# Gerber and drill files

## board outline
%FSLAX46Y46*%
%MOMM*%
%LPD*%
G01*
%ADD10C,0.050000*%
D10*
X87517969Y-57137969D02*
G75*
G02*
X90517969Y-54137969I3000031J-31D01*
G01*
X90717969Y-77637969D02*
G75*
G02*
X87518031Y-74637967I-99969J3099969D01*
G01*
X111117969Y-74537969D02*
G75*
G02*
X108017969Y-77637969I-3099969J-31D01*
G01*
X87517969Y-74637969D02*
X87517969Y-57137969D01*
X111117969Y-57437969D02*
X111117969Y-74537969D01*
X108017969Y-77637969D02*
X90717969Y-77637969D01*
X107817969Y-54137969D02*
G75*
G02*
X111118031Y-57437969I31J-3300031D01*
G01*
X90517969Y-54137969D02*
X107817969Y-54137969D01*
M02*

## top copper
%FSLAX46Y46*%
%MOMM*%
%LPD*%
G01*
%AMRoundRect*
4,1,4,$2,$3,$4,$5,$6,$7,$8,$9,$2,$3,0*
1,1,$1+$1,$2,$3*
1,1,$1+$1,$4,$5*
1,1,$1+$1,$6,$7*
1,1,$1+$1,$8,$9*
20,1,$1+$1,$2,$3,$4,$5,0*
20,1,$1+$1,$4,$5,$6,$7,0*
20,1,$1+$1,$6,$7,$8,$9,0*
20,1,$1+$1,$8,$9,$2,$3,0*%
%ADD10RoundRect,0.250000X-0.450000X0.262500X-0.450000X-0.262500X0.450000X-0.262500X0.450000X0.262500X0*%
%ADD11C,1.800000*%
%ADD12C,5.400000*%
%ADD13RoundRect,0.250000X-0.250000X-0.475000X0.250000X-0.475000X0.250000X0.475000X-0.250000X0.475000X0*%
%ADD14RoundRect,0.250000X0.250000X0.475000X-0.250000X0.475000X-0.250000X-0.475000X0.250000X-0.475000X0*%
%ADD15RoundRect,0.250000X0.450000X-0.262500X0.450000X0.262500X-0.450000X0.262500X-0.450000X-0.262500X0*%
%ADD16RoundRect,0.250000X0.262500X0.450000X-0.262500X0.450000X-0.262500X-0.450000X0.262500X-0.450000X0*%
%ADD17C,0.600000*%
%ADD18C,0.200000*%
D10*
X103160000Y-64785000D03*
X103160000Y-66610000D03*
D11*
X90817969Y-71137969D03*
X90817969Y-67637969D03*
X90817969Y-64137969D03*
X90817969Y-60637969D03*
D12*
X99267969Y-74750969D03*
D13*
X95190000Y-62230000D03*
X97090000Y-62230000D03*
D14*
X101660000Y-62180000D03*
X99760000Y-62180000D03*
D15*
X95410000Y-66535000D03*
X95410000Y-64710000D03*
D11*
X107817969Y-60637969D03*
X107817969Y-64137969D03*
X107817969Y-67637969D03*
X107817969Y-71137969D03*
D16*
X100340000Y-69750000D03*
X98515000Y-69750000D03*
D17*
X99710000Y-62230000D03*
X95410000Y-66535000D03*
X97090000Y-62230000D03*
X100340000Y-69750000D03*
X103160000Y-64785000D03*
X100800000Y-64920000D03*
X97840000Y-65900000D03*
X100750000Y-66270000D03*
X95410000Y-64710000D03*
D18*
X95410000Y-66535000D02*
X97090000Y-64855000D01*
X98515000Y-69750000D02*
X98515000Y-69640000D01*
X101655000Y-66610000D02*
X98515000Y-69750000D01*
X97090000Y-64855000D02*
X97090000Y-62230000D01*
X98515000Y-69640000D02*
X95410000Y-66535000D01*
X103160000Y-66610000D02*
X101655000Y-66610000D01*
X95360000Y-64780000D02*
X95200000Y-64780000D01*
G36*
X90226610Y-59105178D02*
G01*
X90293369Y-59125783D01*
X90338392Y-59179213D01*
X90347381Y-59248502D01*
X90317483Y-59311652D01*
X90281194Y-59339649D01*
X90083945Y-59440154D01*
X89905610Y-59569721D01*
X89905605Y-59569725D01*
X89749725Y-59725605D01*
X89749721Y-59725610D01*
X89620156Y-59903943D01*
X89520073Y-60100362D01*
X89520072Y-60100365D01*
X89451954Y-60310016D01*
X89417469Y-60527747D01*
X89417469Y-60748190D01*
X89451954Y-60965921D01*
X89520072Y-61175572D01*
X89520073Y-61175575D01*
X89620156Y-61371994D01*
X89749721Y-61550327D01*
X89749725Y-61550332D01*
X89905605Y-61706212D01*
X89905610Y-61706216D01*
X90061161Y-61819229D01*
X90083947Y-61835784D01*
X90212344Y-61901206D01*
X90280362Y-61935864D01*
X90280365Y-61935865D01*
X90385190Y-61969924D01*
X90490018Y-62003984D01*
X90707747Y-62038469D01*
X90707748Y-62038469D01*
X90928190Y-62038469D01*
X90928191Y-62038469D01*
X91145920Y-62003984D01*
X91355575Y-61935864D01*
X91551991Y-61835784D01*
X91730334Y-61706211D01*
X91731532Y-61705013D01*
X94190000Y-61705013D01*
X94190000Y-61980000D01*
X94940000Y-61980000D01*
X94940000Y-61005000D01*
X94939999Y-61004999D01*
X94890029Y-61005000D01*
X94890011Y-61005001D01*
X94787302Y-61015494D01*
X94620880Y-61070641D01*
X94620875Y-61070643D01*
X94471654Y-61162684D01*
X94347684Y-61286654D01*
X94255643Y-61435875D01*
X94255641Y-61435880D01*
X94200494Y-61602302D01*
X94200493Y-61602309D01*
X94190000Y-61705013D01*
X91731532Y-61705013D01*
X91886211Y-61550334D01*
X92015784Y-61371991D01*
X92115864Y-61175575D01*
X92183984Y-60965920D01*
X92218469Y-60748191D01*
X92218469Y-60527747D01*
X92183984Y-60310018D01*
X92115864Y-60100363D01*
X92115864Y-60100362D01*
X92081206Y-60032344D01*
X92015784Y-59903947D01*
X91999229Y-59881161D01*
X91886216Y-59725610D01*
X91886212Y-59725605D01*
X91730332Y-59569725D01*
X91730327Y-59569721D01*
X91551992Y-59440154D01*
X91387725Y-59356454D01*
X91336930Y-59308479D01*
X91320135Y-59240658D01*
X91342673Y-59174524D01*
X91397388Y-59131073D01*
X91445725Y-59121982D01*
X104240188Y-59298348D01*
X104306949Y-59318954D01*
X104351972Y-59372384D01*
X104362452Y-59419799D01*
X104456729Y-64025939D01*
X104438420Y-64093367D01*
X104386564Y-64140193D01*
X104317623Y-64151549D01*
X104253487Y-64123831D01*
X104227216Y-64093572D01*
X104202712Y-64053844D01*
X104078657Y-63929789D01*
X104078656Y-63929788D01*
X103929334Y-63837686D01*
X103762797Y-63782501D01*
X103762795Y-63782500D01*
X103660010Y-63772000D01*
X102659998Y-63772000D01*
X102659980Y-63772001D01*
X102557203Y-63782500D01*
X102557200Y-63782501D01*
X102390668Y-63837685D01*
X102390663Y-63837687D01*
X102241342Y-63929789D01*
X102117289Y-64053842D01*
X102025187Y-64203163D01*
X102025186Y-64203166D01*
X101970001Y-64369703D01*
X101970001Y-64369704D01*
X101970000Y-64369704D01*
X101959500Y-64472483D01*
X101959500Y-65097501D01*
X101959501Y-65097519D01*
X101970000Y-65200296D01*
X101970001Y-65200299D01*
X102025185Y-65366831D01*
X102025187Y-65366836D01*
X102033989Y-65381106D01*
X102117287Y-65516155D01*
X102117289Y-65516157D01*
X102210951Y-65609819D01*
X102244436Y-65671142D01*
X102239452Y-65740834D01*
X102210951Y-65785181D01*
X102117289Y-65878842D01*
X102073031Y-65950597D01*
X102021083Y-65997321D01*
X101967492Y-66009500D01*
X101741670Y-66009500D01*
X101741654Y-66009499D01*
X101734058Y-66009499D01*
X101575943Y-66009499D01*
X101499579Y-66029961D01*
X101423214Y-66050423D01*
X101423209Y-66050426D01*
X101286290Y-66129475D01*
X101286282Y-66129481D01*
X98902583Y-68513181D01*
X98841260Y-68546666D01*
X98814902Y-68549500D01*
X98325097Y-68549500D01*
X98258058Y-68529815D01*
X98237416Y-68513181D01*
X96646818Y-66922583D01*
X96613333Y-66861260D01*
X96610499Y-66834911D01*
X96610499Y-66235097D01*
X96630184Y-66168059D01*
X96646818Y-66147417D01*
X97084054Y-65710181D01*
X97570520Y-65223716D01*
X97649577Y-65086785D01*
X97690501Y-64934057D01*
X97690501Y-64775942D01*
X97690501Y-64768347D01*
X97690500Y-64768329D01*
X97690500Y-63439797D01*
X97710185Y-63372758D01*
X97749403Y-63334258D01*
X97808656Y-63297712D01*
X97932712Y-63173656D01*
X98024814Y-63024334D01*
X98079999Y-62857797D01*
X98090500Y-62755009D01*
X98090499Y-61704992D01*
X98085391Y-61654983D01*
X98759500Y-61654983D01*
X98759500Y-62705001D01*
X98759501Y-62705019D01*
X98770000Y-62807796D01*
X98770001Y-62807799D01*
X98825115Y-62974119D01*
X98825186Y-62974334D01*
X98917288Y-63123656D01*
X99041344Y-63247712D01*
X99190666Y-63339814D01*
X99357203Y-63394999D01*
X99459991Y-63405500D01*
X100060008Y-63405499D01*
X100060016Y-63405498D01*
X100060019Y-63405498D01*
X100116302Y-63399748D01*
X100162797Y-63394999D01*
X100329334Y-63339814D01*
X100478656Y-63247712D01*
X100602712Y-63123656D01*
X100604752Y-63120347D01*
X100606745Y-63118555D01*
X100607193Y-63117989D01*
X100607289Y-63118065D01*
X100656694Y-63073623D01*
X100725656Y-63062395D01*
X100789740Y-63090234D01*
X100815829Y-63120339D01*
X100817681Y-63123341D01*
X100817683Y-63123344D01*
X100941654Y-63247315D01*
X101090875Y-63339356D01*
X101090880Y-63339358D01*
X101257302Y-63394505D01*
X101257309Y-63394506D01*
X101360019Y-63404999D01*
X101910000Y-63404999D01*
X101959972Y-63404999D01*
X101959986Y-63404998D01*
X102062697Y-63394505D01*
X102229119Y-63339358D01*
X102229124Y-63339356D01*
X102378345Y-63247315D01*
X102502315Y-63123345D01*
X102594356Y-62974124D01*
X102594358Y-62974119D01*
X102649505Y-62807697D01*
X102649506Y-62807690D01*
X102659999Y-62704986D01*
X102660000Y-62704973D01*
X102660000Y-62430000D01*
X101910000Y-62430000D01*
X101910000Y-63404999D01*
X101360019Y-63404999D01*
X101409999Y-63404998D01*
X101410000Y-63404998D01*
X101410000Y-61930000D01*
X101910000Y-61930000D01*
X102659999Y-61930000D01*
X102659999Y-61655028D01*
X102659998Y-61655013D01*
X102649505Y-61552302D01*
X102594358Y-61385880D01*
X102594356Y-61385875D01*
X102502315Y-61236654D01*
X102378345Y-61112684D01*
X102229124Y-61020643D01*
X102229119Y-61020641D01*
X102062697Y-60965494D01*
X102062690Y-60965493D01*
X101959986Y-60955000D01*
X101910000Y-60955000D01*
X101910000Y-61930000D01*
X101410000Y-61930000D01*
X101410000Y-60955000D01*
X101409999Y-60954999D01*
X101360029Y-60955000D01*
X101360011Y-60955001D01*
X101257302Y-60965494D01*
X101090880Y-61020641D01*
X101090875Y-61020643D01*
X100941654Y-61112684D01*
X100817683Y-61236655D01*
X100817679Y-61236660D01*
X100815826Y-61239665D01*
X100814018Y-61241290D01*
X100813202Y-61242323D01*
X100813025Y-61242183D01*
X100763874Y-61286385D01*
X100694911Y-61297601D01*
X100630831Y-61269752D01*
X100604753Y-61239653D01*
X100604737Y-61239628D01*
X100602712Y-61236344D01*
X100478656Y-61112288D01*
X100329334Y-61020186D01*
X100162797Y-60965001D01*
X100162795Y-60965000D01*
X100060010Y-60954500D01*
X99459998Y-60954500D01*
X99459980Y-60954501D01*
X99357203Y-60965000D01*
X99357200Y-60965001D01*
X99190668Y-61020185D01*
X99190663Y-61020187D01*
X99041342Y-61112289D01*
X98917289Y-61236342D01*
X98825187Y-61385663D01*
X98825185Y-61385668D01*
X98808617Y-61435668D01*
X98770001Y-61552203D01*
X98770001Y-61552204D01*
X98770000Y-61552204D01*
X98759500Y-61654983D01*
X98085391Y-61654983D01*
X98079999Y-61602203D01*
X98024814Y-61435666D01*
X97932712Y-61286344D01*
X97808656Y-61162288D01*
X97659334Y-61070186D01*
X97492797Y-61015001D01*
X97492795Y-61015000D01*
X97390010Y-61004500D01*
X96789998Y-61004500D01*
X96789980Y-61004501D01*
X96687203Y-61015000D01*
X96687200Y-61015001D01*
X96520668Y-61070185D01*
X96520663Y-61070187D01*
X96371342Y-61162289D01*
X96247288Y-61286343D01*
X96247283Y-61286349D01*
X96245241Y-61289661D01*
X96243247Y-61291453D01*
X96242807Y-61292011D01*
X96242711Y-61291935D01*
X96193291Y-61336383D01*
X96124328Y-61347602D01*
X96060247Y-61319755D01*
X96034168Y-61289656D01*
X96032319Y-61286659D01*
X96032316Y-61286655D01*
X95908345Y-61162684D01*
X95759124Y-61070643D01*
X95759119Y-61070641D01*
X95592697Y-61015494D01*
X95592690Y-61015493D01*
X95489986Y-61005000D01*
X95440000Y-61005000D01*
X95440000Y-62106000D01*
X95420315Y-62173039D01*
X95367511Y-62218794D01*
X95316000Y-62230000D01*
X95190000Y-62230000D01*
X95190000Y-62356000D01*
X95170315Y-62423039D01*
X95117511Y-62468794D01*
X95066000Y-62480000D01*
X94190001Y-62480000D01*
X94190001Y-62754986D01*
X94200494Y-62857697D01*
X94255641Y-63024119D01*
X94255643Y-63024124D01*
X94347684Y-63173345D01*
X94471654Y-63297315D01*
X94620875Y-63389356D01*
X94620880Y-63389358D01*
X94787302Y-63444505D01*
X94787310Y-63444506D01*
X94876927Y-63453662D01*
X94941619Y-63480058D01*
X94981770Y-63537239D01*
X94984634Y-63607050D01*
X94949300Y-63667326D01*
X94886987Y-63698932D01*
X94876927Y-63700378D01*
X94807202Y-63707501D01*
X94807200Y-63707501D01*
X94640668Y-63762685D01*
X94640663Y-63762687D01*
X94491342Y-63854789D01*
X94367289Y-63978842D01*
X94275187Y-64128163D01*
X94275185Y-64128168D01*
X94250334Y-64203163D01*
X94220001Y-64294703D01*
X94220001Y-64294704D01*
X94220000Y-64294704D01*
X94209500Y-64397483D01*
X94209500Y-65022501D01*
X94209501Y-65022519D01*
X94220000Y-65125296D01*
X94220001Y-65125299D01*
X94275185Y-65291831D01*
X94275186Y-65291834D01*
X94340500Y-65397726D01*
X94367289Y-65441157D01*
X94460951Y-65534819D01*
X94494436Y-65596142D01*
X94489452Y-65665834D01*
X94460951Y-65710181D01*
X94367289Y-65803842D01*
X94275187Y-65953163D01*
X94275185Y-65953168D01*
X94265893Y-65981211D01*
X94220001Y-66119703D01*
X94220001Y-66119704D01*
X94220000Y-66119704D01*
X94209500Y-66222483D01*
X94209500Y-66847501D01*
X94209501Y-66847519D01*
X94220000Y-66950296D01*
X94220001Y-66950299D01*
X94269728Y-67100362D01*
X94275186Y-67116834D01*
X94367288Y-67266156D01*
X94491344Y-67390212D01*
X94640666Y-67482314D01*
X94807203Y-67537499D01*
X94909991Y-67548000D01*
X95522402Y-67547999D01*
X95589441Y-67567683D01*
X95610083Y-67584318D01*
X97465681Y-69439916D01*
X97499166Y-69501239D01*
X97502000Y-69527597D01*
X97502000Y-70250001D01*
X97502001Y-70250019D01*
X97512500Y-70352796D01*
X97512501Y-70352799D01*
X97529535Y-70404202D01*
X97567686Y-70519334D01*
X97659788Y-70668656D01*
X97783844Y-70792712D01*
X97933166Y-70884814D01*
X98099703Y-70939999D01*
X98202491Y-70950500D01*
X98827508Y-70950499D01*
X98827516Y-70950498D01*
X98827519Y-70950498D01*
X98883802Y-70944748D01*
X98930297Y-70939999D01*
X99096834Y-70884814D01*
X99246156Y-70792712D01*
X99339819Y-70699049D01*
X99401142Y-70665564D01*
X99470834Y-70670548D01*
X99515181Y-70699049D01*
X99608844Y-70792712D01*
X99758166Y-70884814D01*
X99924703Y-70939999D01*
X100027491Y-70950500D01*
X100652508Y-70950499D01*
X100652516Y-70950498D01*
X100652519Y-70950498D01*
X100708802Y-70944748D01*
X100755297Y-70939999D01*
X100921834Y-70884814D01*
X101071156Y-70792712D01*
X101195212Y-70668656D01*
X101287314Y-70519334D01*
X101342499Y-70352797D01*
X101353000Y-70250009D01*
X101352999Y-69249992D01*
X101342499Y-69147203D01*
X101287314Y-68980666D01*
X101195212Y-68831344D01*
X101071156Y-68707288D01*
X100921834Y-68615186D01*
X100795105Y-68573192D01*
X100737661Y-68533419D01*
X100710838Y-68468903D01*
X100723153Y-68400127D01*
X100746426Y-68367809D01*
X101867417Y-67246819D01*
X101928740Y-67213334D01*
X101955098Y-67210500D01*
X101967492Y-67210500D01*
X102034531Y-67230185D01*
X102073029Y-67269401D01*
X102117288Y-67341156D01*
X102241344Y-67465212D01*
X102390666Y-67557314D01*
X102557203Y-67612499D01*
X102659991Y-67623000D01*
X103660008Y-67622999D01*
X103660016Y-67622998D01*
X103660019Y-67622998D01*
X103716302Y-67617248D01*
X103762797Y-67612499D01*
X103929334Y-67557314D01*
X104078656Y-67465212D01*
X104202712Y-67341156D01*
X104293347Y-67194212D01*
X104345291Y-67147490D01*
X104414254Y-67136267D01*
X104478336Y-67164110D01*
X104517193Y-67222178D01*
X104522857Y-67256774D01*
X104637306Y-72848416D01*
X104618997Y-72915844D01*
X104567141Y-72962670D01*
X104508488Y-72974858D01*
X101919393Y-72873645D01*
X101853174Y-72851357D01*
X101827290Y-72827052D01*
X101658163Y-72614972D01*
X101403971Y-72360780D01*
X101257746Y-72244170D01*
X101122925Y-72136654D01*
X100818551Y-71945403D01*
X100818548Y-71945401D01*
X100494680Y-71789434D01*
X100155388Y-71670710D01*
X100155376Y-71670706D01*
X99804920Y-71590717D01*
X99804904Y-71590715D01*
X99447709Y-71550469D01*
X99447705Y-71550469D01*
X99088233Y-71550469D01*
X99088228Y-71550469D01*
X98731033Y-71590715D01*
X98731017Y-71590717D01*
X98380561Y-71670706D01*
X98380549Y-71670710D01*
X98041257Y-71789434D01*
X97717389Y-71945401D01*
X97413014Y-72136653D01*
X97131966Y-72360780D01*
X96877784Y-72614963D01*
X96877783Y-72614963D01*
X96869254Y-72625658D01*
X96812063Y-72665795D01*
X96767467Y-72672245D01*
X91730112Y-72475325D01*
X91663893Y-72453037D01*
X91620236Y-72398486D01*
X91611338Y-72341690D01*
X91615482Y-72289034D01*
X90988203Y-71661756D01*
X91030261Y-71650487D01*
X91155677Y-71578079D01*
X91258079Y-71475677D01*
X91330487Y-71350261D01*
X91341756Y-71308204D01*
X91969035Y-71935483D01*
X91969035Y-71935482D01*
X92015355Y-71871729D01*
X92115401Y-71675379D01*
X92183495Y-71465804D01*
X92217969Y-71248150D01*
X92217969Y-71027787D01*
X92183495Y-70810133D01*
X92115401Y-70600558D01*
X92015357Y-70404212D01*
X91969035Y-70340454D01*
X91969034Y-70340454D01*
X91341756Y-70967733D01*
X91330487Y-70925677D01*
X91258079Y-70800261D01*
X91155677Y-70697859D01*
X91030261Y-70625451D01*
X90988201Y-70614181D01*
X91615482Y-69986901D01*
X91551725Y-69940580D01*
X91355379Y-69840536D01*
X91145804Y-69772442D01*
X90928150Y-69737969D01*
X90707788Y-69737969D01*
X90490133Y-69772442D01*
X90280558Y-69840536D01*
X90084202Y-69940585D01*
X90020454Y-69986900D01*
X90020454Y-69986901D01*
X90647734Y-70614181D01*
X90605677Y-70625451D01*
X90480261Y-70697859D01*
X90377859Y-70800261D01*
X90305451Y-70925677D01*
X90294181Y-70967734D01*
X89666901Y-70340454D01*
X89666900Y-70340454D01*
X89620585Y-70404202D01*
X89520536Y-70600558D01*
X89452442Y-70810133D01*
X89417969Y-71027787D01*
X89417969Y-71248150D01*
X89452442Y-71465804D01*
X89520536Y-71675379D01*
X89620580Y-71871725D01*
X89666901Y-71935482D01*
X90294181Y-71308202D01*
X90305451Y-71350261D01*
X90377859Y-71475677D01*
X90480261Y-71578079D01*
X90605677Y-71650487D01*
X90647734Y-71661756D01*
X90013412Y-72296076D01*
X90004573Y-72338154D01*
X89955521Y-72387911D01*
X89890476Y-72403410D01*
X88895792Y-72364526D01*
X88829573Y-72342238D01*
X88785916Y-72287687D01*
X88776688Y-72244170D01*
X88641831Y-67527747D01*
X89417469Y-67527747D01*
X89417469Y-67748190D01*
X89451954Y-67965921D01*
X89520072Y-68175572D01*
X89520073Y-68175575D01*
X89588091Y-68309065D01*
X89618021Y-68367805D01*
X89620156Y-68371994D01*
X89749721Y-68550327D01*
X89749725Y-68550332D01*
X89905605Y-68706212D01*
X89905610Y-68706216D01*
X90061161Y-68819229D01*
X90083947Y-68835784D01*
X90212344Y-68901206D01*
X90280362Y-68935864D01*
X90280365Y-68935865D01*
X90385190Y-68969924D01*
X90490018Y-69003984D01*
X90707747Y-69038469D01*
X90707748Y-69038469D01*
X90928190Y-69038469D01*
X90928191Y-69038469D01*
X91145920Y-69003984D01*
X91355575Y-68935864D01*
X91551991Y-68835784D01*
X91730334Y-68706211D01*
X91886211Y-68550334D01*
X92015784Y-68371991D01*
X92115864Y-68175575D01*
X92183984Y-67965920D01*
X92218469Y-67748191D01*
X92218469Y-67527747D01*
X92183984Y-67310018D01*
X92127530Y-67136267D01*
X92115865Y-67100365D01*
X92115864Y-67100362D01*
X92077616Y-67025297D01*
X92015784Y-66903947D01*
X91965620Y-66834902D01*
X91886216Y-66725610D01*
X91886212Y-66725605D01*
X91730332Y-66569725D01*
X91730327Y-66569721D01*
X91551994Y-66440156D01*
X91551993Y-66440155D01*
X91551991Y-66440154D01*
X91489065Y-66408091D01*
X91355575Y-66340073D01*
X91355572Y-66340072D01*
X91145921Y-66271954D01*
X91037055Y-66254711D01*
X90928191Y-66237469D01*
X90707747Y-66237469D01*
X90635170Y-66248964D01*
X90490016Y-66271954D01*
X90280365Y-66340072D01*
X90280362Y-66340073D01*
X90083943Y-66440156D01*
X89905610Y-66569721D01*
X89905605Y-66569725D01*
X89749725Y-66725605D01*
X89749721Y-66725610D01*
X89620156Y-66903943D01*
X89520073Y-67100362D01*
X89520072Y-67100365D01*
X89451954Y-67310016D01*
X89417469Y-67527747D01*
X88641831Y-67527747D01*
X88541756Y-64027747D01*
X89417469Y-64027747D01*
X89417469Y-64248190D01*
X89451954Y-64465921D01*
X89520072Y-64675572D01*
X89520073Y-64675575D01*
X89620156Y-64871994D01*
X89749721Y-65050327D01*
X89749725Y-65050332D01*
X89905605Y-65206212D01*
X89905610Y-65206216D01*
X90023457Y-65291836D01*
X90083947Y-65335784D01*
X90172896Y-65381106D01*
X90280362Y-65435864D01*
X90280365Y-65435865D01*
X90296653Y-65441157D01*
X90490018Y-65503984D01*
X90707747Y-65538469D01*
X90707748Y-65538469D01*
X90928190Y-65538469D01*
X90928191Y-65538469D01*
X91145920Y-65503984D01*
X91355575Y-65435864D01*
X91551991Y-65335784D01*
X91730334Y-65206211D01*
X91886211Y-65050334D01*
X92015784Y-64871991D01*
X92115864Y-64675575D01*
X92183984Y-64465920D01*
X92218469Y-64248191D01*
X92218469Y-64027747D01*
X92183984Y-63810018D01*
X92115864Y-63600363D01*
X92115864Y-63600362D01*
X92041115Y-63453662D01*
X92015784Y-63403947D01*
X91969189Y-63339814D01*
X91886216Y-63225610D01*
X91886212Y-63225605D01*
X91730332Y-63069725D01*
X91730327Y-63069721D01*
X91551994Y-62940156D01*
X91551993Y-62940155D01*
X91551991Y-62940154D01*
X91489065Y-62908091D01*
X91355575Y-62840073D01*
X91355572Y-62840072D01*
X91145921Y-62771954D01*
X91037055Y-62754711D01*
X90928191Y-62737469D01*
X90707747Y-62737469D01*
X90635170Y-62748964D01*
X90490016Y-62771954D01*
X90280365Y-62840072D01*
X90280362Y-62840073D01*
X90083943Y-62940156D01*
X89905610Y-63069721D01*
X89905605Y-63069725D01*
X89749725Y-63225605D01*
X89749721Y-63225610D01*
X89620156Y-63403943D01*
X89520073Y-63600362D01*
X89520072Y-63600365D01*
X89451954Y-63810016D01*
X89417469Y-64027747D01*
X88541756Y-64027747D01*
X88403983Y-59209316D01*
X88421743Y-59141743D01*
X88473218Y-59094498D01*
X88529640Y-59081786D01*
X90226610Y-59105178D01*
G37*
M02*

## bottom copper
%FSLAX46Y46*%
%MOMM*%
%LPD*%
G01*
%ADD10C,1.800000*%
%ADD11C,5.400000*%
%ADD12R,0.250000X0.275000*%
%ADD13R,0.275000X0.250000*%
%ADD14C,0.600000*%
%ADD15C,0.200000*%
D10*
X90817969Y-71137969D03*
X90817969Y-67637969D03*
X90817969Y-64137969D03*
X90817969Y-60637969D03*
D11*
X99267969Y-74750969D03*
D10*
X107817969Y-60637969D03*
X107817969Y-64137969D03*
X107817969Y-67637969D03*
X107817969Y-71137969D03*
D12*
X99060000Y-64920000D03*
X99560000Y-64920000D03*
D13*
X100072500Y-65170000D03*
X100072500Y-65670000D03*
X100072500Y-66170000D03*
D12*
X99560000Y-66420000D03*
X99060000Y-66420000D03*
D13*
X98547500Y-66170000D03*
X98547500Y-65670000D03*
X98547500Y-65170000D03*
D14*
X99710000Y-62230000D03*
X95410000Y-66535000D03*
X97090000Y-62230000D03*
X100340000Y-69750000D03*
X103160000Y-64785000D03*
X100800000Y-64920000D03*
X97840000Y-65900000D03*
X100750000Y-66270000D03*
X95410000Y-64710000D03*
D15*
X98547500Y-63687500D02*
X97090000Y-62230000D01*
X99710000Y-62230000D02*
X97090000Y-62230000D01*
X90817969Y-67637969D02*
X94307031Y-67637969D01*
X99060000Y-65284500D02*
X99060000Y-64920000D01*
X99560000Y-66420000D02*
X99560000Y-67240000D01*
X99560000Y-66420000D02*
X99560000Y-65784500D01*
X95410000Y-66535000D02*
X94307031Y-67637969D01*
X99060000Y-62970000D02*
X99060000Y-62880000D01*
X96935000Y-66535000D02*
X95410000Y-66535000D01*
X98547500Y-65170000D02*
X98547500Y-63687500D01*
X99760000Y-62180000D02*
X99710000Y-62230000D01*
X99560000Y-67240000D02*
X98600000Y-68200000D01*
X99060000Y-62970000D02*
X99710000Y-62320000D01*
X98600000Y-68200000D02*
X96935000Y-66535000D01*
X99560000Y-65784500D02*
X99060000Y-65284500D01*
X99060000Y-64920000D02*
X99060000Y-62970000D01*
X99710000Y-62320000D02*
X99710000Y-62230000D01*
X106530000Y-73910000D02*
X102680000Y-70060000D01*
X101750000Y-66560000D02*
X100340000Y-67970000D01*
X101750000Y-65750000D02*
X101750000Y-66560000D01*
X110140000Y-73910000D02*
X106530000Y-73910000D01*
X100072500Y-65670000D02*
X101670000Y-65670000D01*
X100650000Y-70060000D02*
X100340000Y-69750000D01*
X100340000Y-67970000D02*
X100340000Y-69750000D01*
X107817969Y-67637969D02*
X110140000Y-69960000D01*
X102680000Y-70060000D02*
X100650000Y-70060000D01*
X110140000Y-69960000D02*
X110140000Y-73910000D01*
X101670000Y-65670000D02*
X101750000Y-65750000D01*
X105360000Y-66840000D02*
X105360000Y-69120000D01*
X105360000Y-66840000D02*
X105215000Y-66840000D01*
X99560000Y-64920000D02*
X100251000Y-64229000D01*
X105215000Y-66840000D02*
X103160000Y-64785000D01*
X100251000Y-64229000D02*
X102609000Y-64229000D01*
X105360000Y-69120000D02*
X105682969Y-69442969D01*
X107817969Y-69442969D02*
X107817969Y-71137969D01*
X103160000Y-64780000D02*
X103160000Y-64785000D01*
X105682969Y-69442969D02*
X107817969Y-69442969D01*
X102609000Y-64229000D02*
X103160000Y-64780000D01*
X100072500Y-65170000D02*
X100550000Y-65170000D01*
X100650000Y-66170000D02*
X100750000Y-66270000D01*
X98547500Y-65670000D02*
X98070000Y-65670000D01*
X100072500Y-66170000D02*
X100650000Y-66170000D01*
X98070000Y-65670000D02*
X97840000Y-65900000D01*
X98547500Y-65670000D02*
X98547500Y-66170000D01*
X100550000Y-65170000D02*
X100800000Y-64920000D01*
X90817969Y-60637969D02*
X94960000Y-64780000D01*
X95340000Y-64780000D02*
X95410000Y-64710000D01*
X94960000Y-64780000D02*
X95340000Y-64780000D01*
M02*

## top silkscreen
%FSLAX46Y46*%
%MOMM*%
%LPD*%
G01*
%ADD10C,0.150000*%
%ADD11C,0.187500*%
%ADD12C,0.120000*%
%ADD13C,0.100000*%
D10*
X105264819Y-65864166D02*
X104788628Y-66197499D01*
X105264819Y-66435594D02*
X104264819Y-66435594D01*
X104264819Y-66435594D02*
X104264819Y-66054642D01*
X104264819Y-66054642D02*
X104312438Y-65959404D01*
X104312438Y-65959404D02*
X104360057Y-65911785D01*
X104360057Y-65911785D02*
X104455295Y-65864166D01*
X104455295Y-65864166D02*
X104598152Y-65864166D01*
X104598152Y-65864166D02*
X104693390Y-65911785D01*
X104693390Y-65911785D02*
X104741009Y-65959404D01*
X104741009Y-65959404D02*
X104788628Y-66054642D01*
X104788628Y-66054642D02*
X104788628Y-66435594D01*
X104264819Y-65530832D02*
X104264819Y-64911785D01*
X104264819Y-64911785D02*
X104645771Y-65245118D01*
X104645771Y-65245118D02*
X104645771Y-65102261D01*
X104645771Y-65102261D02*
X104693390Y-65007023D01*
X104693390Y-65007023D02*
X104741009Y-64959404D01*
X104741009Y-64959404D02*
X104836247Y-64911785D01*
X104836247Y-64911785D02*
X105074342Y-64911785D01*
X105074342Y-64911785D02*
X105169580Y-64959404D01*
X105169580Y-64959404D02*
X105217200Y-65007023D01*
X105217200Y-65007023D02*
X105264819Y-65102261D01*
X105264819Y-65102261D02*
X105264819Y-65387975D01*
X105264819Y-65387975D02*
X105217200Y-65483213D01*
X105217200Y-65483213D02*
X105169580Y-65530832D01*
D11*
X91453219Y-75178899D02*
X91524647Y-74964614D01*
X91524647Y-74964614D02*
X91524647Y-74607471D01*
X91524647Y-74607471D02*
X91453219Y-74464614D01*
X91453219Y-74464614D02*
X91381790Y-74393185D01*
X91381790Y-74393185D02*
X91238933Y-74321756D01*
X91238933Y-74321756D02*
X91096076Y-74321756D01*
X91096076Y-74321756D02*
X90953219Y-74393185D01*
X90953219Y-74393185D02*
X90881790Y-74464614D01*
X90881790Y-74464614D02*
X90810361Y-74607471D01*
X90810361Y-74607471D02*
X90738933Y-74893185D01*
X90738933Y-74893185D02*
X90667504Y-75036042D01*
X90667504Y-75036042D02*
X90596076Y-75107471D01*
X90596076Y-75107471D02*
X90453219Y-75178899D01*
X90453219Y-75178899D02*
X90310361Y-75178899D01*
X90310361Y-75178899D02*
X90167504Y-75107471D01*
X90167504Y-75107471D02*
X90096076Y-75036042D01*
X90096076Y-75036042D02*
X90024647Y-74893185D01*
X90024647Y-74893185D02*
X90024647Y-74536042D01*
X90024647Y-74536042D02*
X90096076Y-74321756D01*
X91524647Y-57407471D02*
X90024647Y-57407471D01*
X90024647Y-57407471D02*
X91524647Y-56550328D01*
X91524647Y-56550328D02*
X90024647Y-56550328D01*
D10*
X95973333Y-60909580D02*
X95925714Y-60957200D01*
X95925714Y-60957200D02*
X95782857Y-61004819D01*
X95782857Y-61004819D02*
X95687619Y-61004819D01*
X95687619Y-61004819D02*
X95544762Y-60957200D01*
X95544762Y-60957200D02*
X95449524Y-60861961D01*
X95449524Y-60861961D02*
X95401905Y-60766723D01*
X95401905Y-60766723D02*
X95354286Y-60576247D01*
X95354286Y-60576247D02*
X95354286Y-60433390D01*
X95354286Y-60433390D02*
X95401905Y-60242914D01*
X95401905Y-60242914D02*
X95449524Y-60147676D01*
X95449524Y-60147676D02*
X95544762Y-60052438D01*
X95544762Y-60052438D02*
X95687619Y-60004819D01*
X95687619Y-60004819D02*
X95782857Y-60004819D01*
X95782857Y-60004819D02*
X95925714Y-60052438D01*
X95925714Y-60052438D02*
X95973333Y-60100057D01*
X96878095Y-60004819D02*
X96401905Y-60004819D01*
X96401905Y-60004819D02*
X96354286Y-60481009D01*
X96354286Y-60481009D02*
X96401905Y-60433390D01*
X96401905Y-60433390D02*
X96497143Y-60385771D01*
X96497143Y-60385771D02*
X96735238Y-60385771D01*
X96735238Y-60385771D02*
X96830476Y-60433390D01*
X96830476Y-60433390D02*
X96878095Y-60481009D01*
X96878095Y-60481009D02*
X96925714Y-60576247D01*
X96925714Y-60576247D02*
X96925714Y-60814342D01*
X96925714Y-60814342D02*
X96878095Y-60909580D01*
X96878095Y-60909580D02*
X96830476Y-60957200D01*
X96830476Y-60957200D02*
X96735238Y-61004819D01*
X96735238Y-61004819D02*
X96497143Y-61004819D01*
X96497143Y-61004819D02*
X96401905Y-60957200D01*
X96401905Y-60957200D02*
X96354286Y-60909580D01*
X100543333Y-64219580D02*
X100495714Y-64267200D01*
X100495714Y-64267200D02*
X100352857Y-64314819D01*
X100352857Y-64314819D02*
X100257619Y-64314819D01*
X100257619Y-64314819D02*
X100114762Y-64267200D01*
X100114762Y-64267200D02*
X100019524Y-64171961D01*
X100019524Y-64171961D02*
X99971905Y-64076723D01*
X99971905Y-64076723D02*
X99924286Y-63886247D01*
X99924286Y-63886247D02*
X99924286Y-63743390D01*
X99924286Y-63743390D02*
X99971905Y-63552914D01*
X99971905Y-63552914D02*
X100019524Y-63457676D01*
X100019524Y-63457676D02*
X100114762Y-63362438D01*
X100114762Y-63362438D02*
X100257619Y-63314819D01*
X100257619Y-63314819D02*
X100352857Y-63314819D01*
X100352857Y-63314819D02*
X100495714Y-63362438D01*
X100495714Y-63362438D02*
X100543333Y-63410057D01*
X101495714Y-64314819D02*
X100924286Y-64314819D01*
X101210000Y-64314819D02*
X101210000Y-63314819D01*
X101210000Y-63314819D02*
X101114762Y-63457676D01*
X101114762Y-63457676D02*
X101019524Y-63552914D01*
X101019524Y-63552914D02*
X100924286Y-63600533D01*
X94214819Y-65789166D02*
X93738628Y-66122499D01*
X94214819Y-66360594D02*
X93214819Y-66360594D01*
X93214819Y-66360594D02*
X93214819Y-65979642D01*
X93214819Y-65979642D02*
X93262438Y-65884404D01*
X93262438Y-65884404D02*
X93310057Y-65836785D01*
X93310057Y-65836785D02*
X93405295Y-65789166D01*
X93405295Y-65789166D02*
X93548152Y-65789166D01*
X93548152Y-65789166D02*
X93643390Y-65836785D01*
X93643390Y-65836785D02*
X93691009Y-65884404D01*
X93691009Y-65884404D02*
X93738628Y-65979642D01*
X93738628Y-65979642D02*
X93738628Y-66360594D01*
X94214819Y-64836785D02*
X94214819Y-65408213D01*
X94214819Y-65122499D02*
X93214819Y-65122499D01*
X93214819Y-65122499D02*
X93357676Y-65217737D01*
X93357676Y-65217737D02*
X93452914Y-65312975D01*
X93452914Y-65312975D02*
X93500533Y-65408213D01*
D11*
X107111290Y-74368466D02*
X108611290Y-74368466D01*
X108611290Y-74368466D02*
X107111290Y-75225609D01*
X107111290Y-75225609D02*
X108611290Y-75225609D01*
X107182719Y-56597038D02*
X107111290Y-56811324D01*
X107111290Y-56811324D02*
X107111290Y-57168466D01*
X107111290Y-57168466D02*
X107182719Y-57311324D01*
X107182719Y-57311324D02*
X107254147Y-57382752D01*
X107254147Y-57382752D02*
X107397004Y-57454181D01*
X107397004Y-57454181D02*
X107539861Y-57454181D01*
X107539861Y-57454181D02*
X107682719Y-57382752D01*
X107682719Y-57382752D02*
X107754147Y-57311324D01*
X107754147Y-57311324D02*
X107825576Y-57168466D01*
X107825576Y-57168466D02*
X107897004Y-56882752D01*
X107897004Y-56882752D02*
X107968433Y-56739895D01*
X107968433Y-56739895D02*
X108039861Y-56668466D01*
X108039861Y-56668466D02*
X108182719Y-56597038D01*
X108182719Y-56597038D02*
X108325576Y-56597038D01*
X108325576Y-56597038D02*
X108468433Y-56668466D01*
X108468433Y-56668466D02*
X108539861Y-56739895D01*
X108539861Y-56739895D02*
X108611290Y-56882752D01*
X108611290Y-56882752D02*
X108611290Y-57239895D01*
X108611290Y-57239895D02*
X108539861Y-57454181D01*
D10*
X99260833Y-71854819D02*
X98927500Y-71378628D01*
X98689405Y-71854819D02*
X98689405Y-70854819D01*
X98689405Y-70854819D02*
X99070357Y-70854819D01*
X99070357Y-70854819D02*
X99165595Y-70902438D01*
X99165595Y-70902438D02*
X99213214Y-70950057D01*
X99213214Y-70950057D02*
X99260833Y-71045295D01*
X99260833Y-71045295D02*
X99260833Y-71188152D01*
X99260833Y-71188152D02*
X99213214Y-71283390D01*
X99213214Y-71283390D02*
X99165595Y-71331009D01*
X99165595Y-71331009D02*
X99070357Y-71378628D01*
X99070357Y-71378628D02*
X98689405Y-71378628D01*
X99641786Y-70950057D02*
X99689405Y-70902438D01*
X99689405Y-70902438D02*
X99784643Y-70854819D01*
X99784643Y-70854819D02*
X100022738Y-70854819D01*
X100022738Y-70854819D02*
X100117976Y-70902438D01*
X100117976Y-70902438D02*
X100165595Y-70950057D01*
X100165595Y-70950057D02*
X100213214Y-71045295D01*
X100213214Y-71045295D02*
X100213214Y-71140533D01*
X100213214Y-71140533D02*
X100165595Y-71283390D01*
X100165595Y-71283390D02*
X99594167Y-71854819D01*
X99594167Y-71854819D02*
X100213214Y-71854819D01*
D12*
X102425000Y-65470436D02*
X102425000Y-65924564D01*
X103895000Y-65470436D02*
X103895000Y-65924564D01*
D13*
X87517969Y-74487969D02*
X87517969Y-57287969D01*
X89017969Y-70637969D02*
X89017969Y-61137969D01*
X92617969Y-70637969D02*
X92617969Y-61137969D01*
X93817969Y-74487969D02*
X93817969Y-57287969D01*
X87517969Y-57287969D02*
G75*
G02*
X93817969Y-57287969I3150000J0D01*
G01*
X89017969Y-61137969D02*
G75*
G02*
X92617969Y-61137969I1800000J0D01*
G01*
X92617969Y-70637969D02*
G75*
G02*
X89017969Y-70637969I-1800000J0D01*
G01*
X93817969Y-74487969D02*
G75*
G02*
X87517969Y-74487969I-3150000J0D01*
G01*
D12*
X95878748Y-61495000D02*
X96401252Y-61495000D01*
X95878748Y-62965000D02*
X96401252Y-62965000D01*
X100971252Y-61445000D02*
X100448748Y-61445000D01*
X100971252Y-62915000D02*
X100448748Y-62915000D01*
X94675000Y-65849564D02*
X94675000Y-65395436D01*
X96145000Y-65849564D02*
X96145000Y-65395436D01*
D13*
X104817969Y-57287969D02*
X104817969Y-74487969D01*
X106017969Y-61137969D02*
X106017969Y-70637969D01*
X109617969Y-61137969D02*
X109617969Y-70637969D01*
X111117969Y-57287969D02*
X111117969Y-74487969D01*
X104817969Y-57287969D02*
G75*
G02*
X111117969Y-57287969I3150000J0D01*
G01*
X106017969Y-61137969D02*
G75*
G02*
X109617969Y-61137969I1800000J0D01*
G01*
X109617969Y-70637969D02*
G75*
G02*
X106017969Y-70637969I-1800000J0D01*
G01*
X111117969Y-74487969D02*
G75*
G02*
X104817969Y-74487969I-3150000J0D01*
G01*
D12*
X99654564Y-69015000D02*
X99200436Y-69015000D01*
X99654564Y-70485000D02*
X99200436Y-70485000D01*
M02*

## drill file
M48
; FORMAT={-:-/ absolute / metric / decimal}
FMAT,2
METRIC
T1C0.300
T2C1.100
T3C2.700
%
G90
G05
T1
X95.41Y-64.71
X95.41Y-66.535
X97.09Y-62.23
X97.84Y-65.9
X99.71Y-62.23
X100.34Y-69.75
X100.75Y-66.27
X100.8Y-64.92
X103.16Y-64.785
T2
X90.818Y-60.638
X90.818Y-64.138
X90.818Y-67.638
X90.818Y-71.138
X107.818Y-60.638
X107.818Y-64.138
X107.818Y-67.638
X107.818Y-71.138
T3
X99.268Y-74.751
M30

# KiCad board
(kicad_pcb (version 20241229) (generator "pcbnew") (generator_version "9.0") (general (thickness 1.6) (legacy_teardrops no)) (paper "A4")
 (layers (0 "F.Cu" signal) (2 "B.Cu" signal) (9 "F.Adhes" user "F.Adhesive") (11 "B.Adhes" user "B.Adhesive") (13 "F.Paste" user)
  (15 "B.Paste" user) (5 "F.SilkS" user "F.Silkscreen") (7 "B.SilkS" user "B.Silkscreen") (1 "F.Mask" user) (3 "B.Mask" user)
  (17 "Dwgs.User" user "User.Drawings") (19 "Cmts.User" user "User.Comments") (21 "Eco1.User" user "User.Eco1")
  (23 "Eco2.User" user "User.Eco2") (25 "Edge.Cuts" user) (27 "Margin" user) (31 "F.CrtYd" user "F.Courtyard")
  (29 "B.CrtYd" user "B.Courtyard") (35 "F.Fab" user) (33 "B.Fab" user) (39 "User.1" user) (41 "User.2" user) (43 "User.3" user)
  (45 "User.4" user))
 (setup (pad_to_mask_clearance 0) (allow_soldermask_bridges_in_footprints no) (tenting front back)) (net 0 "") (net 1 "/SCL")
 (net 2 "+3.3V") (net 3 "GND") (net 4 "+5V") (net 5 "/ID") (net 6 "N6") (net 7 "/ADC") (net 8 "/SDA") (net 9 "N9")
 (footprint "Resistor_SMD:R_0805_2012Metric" (layer "F.Cu") (at 103.16 65.6975 -90)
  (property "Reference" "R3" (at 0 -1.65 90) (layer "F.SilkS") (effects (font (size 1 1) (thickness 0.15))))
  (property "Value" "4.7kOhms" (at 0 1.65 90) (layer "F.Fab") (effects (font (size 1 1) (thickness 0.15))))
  (fp_line (start -0.227064 0.735) (end 0.227064 0.735) (stroke (width 0.12) (type solid)) (layer "F.SilkS"))
  (fp_line (start -0.227064 -0.735) (end 0.227064 -0.735) (stroke (width 0.12) (type solid)) (layer "F.SilkS"))
  (pad "1" smd roundrect (at -0.9125 0 270) (size 1.025 1.4) (layers "F.Cu" "F.Mask" "F.Paste") (roundrect_rratio 0.243902) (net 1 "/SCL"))
  (pad "2" smd roundrect (at 0.9125 0 270) (size 1.025 1.4) (layers "F.Cu" "F.Mask" "F.Paste") (roundrect_rratio 0.243902) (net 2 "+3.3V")))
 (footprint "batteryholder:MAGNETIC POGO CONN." (layer "F.Cu") (at 90.817969 65.887969 90)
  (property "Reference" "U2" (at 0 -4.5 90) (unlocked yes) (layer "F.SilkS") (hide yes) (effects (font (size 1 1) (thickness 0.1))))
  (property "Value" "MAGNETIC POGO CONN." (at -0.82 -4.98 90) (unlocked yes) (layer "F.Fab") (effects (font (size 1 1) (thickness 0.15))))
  (fp_line (start -8.6 -3.3) (end 8.6 -3.3) (stroke (width 0.1) (type default)) (layer "F.SilkS"))
  (fp_line (start -4.75 -1.8) (end 4.75 -1.8) (stroke (width 0.1) (type default)) (layer "F.SilkS"))
  (fp_line (start -4.75 1.8) (end 4.75 1.8) (stroke (width 0.1) (type default)) (layer "F.SilkS"))
  (fp_line (start -8.6 3) (end 8.6 3) (stroke (width 0.1) (type default)) (layer "F.SilkS"))
  (fp_arc (start 8.6 -3.3) (mid 11.75 -0.15) (end 8.6 3) (stroke (width 0.1) (type default)) (layer "F.SilkS"))
  (fp_arc (start 4.75 -1.8) (mid 6.55 0) (end 4.75 1.8) (stroke (width 0.1) (type default)) (layer "F.SilkS"))
  (fp_arc (start -4.75 1.8) (mid -6.55 0) (end -4.75 -1.8) (stroke (width 0.1) (type default)) (layer "F.SilkS"))
  (fp_arc (start -8.6 3) (mid -11.75 -0.15) (end -8.6 -3.3) (stroke (width 0.1) (type default)) (layer "F.SilkS"))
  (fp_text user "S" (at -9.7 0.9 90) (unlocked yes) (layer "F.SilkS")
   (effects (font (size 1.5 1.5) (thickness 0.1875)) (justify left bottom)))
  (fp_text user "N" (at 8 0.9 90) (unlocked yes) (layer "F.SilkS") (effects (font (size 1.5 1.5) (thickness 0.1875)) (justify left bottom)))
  (pad "1" thru_hole circle (at -5.25 0 90) (size 1.8 1.8) (drill 1.1) (layers "*.Cu" "*.Mask") (remove_unused_layers no) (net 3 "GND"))
  (pad "2" thru_hole circle (at -1.75 0 90) (size 1.8 1.8) (drill 1.1) (layers "*.Cu" "*.Mask") (remove_unused_layers no) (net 2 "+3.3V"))
  (pad "3" thru_hole circle (at 1.75 0 90) (size 1.8 1.8) (drill 1.1) (layers "*.Cu" "*.Mask") (remove_unused_layers no) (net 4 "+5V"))
  (pad "4" thru_hole circle (at 5.25 0 90) (size 1.8 1.8) (drill 1.1) (layers "*.Cu" "*.Mask") (remove_unused_layers no) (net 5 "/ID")))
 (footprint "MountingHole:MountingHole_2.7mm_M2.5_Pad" (layer "F.Cu") (at 99.267969 74.750969)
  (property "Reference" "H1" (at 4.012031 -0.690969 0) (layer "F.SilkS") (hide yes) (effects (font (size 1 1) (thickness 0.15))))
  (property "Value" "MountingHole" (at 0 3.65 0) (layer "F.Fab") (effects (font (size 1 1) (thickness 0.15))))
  (pad "1" thru_hole circle (at 0 0) (size 5.4 5.4) (drill 2.7) (layers "*.Cu" "*.Mask") (remove_unused_layers no) (zone_connect 2)))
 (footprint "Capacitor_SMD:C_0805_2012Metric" (layer "F.Cu") (at 96.14 62.23)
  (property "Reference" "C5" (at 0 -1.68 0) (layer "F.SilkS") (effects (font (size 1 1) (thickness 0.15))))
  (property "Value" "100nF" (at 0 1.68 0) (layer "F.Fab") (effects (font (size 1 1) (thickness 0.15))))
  (fp_line (start -0.261252 -0.735) (end 0.261252 -0.735) (stroke (width 0.12) (type solid)) (layer "F.SilkS"))
  (fp_line (start -0.261252 0.735) (end 0.261252 0.735) (stroke (width 0.12) (type solid)) (layer "F.SilkS"))
  (pad "1" smd roundrect (at -0.95 0) (size 1 1.45) (layers "F.Cu" "F.Mask" "F.Paste") (roundrect_rratio 0.25) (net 3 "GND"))
  (pad "2" smd roundrect (at 0.95 0) (size 1 1.45) (layers "F.Cu" "F.Mask" "F.Paste") (roundrect_rratio 0.25) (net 2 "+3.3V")))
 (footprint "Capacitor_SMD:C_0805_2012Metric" (layer "F.Cu") (at 100.71 62.18 180)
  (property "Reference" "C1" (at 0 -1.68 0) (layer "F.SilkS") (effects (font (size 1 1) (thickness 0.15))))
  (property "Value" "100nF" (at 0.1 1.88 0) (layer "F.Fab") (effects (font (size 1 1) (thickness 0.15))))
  (fp_line (start -0.261252 0.735) (end 0.261252 0.735) (stroke (width 0.12) (type solid)) (layer "F.SilkS"))
  (fp_line (start -0.261252 -0.735) (end 0.261252 -0.735) (stroke (width 0.12) (type solid)) (layer "F.SilkS"))
  (pad "1" smd roundrect (at -0.95 0 180) (size 1 1.45) (layers "F.Cu" "F.Mask" "F.Paste") (roundrect_rratio 0.25) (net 3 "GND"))
  (pad "2" smd roundrect (at 0.95 0 180) (size 1 1.45) (layers "F.Cu" "F.Mask" "F.Paste") (roundrect_rratio 0.25) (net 2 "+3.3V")))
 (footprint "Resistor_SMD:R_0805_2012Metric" (layer "F.Cu") (at 95.41 65.6225 90)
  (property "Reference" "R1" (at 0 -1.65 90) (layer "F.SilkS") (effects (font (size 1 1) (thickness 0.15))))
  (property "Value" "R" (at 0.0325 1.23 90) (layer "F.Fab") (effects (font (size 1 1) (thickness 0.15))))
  (fp_line (start -0.227064 -0.735) (end 0.227064 -0.735) (stroke (width 0.12) (type solid)) (layer "F.SilkS"))
  (fp_line (start -0.227064 0.735) (end 0.227064 0.735) (stroke (width 0.12) (type solid)) (layer "F.SilkS"))
  (pad "1" smd roundrect (at -0.9125 0 90) (size 1.025 1.4) (layers "F.Cu" "F.Mask" "F.Paste") (roundrect_rratio 0.243902) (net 2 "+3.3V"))
  (pad "2" smd roundrect (at 0.9125 0 90) (size 1.025 1.4) (layers "F.Cu" "F.Mask" "F.Paste") (roundrect_rratio 0.243902) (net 5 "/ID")))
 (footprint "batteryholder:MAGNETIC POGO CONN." (layer "F.Cu") (at 107.817969 65.887969 -90)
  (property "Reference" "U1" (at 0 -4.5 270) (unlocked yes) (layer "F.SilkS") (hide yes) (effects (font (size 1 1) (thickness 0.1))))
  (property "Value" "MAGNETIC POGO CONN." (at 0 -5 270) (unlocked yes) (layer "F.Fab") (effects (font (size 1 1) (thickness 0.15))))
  (fp_line (start -8.6 3) (end 8.6 3) (stroke (width 0.1) (type default)) (layer "F.SilkS"))
  (fp_line (start -4.75 1.8) (end 4.75 1.8) (stroke (width 0.1) (type default)) (layer "F.SilkS"))
  (fp_line (start -4.75 -1.8) (end 4.75 -1.8) (stroke (width 0.1) (type default)) (layer "F.SilkS"))
  (fp_line (start -8.6 -3.3) (end 8.6 -3.3) (stroke (width 0.1) (type default)) (layer "F.SilkS"))
  (fp_arc (start -8.6 3) (mid -11.75 -0.15) (end -8.6 -3.3) (stroke (width 0.1) (type default)) (layer "F.SilkS"))
  (fp_arc (start -4.75 1.8) (mid -6.55 0) (end -4.75 -1.8) (stroke (width 0.1) (type default)) (layer "F.SilkS"))
  (fp_arc (start 4.75 -1.8) (mid 6.55 0) (end 4.75 1.8) (stroke (width 0.1) (type default)) (layer "F.SilkS"))
  (fp_arc (start 8.6 -3.3) (mid 11.75 -0.15) (end 8.6 3) (stroke (width 0.1) (type default)) (layer "F.SilkS"))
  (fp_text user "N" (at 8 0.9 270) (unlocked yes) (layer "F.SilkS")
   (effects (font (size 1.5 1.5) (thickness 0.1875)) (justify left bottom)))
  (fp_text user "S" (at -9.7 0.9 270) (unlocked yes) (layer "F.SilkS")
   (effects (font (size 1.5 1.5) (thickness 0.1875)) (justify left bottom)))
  (pad "1" thru_hole circle (at -5.25 0 270) (size 1.8 1.8) (drill 1.1) (layers "*.Cu" "*.Mask") (remove_unused_layers no) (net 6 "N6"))
  (pad "2" thru_hole circle (at -1.75 0 270) (size 1.8 1.8) (drill 1.1) (layers "*.Cu" "*.Mask") (remove_unused_layers no) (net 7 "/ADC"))
  (pad "3" thru_hole circle (at 1.75 0 270) (size 1.8 1.8) (drill 1.1) (layers "*.Cu" "*.Mask") (remove_unused_layers no) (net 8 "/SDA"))
  (pad "4" thru_hole circle (at 5.25 0 270) (size 1.8 1.8) (drill 1.1) (layers "*.Cu" "*.Mask") (remove_unused_layers no) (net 1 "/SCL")))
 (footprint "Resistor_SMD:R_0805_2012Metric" (layer "F.Cu") (at 99.4275 69.75 180)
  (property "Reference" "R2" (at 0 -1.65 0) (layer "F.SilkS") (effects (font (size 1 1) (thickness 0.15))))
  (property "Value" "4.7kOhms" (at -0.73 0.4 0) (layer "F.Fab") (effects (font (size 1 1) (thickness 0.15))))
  (fp_line (start -0.227064 0.735) (end 0.227064 0.735) (stroke (width 0.12) (type solid)) (layer "F.SilkS"))
  (fp_line (start -0.227064 -0.735) (end 0.227064 -0.735) (stroke (width 0.12) (type solid)) (layer "F.SilkS"))
  (pad "1" smd roundrect (at -0.9125 0 180) (size 1.025 1.4) (layers "F.Cu" "F.Mask" "F.Paste") (roundrect_rratio 0.243902) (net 8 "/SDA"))
  (pad "2" smd roundrect (at 0.9125 0 180) (size 1.025 1.4) (layers "F.Cu" "F.Mask" "F.Paste") (roundrect_rratio 0.243902) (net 2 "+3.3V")))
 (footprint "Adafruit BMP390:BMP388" (layer "B.Cu") (at 99.31 65.67 180)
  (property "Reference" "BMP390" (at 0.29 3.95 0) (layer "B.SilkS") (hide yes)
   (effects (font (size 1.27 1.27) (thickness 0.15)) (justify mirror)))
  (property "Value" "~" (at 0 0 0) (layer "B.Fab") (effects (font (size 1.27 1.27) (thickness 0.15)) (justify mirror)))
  (pad "1" smd rect (at 0.25 0.75) (size 0.25 0.275) (layers "B.Cu" "B.Mask" "B.Paste") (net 2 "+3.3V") (solder_mask_margin 0.0508)
   (solder_paste_margin 0) (thermal_bridge_angle 0))
  (pad "2" smd rect (at -0.25 0.75) (size 0.25 0.275) (layers "B.Cu" "B.Mask" "B.Paste") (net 1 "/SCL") (solder_mask_margin 0.0508)
   (solder_paste_margin 0) (thermal_bridge_angle 0))
  (pad "3" smd rect (at -0.7625 0.5 90) (size 0.25 0.275) (layers "B.Cu" "B.Mask" "B.Paste") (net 3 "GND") (solder_mask_margin 0.0508)
   (solder_paste_margin 0) (thermal_bridge_angle 0))
  (pad "4" smd rect (at -0.7625 0 90) (size 0.25 0.275) (layers "B.Cu" "B.Mask" "B.Paste") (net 8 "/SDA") (solder_mask_margin 0.0508)
   (solder_paste_margin 0) (thermal_bridge_angle 0))
  (pad "5" smd rect (at -0.7625 -0.5 90) (size 0.25 0.275) (layers "B.Cu" "B.Mask" "B.Paste") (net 3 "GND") (solder_mask_margin 0.0508)
   (solder_paste_margin 0) (thermal_bridge_angle 0))
  (pad "6" smd rect (at -0.25 -0.75) (size 0.25 0.275) (layers "B.Cu" "B.Mask" "B.Paste") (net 2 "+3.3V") (solder_mask_margin 0.0508)
   (solder_paste_margin 0) (thermal_bridge_angle 0))
  (pad "7" smd rect (at 0.25 -0.75) (size 0.25 0.275) (layers "B.Cu" "B.Mask" "B.Paste") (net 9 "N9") (solder_mask_margin 0.0508)
   (solder_paste_margin 0) (thermal_bridge_angle 0))
  (pad "8" smd rect (at 0.7625 -0.5 90) (size 0.25 0.275) (layers "B.Cu" "B.Mask" "B.Paste") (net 3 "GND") (solder_mask_margin 0.0508)
   (solder_paste_margin 0) (thermal_bridge_angle 0))
  (pad "9" smd rect (at 0.7625 0 90) (size 0.25 0.275) (layers "B.Cu" "B.Mask" "B.Paste") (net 3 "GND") (solder_mask_margin 0.0508)
   (solder_paste_margin 0) (thermal_bridge_angle 0))
  (pad "10" smd rect (at 0.7625 0.5 90) (size 0.25 0.275) (layers "B.Cu" "B.Mask" "B.Paste") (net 2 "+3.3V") (solder_mask_margin 0.0508)
   (solder_paste_margin 0) (thermal_bridge_angle 0)))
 (gr_arc (start 87.517969 57.137969) (mid 88.396649 55.016649) (end 90.517969 54.137969) (stroke (width 0.05) (type default))
  (layer "Edge.Cuts"))
 (gr_arc (start 90.717969 77.637969) (mid 88.496649 76.800711) (end 87.517969 74.637969) (stroke (width 0.05) (type default))
  (layer "Edge.Cuts"))
 (gr_arc (start 111.117969 74.537969) (mid 110.21 76.73) (end 108.017969 77.637969) (stroke (width 0.05) (type default)) (layer "Edge.Cuts"))
 (gr_line (start 87.517969 74.637969) (end 87.517969 57.137969) (stroke (width 0.05) (type default)) (layer "Edge.Cuts"))
 (gr_line (start 111.117969 57.437969) (end 111.117969 74.537969) (stroke (width 0.05) (type default)) (layer "Edge.Cuts"))
 (gr_line (start 108.017969 77.637969) (end 90.717969 77.637969) (stroke (width 0.05) (type solid)) (layer "Edge.Cuts"))
 (gr_arc (start 107.817969 54.137969) (mid 110.151421 55.104517) (end 111.117969 57.437969) (stroke (width 0.05) (type default))
  (layer "Edge.Cuts"))
 (gr_line (start 90.517969 54.137969) (end 107.817969 54.137969) (stroke (width 0.05) (type default)) (layer "Edge.Cuts"))
 (segment (start 95.41 66.535) (end 97.09 64.855) (width 0.2) (layer "F.Cu") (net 2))
 (segment (start 98.515 69.75) (end 98.515 69.64) (width 0.2) (layer "F.Cu") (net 2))
 (segment (start 101.655 66.61) (end 98.515 69.75) (width 0.2) (layer "F.Cu") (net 2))
 (segment (start 97.09 64.855) (end 97.09 62.23) (width 0.2) (layer "F.Cu") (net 2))
 (segment (start 98.515 69.64) (end 95.41 66.535) (width 0.2) (layer "F.Cu") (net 2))
 (segment (start 103.16 66.61) (end 101.655 66.61) (width 0.2) (layer "F.Cu") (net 2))
 (via blind (at 99.71 62.23) (size 0.6) (drill 0.3) (layers "F.Cu" "B.Cu") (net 2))
 (via blind (at 95.41 66.535) (size 0.6) (drill 0.3) (layers "F.Cu" "B.Cu") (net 2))
 (via blind (at 97.09 62.23) (size 0.6) (drill 0.3) (layers "F.Cu" "B.Cu") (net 2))
 (segment (start 98.5475 63.6875) (end 97.09 62.23) (width 0.2) (layer "B.Cu") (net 2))
 (segment (start 99.71 62.23) (end 97.09 62.23) (width 0.2) (layer "B.Cu") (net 2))
 (segment (start 90.817969 67.637969) (end 94.307031 67.637969) (width 0.2) (layer "B.Cu") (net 2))
 (segment (start 99.06 65.2845) (end 99.06 64.92) (width 0.2) (layer "B.Cu") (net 2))
 (segment (start 99.56 66.42) (end 99.56 67.24) (width 0.2) (layer "B.Cu") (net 2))
 (segment (start 99.56 66.42) (end 99.56 65.7845) (width 0.2) (layer "B.Cu") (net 2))
 (segment (start 95.41 66.535) (end 94.307031 67.637969) (width 0.2) (layer "B.Cu") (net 2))
 (segment (start 99.06 62.97) (end 99.06 62.88) (width 0.2) (layer "B.Cu") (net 2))
 (segment (start 96.935 66.535) (end 95.41 66.535) (width 0.2) (layer "B.Cu") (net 2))
 (segment (start 98.5475 65.17) (end 98.5475 63.6875) (width 0.2) (layer "B.Cu") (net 2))
 (segment (start 99.76 62.18) (end 99.71 62.23) (width 0.2) (layer "B.Cu") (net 2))
 (segment (start 99.56 67.24) (end 98.6 68.2) (width 0.2) (layer "B.Cu") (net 2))
 (segment (start 99.06 62.97) (end 99.71 62.32) (width 0.2) (layer "B.Cu") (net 2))
 (segment (start 98.6 68.2) (end 96.935 66.535) (width 0.2) (layer "B.Cu") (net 2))
 (segment (start 99.56 65.7845) (end 99.06 65.2845) (width 0.2) (layer "B.Cu") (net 2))
 (segment (start 99.06 64.92) (end 99.06 62.97) (width 0.2) (layer "B.Cu") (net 2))
 (segment (start 99.71 62.32) (end 99.71 62.23) (width 0.2) (layer "B.Cu") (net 2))
 (via blind (at 100.34 69.75) (size 0.6) (drill 0.3) (layers "F.Cu" "B.Cu") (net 8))
 (segment (start 106.53 73.91) (end 102.68 70.06) (width 0.2) (layer "B.Cu") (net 8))
 (segment (start 101.75 66.56) (end 100.34 67.97) (width 0.2) (layer "B.Cu") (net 8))
 (segment (start 101.75 65.75) (end 101.75 66.56) (width 0.2) (layer "B.Cu") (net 8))
 (segment (start 110.14 73.91) (end 106.53 73.91) (width 0.2) (layer "B.Cu") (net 8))
 (segment (start 100.0725 65.67) (end 101.67 65.67) (width 0.2) (layer "B.Cu") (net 8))
 (segment (start 100.65 70.06) (end 100.34 69.75) (width 0.2) (layer "B.Cu") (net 8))
 (segment (start 100.34 67.97) (end 100.34 69.75) (width 0.2) (layer "B.Cu") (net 8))
 (segment (start 107.817969 67.637969) (end 110.14 69.96) (width 0.2) (layer "B.Cu") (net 8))
 (segment (start 102.68 70.06) (end 100.65 70.06) (width 0.2) (layer "B.Cu") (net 8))
 (segment (start 110.14 69.96) (end 110.14 73.91) (width 0.2) (layer "B.Cu") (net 8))
 (segment (start 101.67 65.67) (end 101.75 65.75) (width 0.2) (layer "B.Cu") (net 8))
 (via blind (at 103.16 64.785) (size 0.6) (drill 0.3) (layers "F.Cu" "B.Cu") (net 1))
 (segment (start 105.36 66.84) (end 105.36 69.12) (width 0.2) (layer "B.Cu") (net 1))
 (segment (start 105.36 66.84) (end 105.215 66.84) (width 0.2) (layer "B.Cu") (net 1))
 (segment (start 99.56 64.92) (end 100.251 64.229) (width 0.2) (layer "B.Cu") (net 1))
 (segment (start 105.215 66.84) (end 103.16 64.785) (width 0.2) (layer "B.Cu") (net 1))
 (segment (start 100.251 64.229) (end 102.609 64.229) (width 0.2) (layer "B.Cu") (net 1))
 (segment (start 105.36 69.12) (end 105.682969 69.442969) (width 0.2) (layer "B.Cu") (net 1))
 (segment (start 107.817969 69.442969) (end 107.817969 71.137969) (width 0.2) (layer "B.Cu") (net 1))
 (segment (start 103.16 64.78) (end 103.16 64.785) (width 0.2) (layer "B.Cu") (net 1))
 (segment (start 105.682969 69.442969) (end 107.817969 69.442969) (width 0.2) (layer "B.Cu") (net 1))
 (segment (start 102.609 64.229) (end 103.16 64.78) (width 0.2) (layer "B.Cu") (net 1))
 (via blind (at 100.8 64.92) (size 0.6) (drill 0.3) (layers "F.Cu" "B.Cu") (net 3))
 (via blind (at 97.84 65.9) (size 0.6) (drill 0.3) (layers "F.Cu" "B.Cu") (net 3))
 (via blind (at 100.75 66.27) (size 0.6) (drill 0.3) (layers "F.Cu" "B.Cu") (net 3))
 (segment (start 100.0725 65.17) (end 100.55 65.17) (width 0.2) (layer "B.Cu") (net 3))
 (segment (start 100.65 66.17) (end 100.75 66.27) (width 0.2) (layer "B.Cu") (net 3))
 (segment (start 98.5475 65.67) (end 98.07 65.67) (width 0.2) (layer "B.Cu") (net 3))
 (segment (start 100.0725 66.17) (end 100.65 66.17) (width 0.2) (layer "B.Cu") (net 3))
 (segment (start 98.07 65.67) (end 97.84 65.9) (width 0.2) (layer "B.Cu") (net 3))
 (segment (start 98.5475 65.67) (end 98.5475 66.17) (width 0.2) (layer "B.Cu") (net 3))
 (segment (start 100.55 65.17) (end 100.8 64.92) (width 0.2) (layer "B.Cu") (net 3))
 (segment (start 95.36 64.78) (end 95.2 64.78) (width 0.2) (layer "F.Cu") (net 5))
 (via blind (at 95.41 64.71) (size 0.6) (drill 0.3) (layers "F.Cu" "B.Cu") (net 5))
 (segment (start 90.817969 60.637969) (end 94.96 64.78) (width 0.2) (layer "B.Cu") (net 5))
 (segment (start 95.34 64.78) (end 95.41 64.71) (width 0.2) (layer "B.Cu") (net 5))
 (segment (start 94.96 64.78) (end 95.34 64.78) (width 0.2) (layer "B.Cu") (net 5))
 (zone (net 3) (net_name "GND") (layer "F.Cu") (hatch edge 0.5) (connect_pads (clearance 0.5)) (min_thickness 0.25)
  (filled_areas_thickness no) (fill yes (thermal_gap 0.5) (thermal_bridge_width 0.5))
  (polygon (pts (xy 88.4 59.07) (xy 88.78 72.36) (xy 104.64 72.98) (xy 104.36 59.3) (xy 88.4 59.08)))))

